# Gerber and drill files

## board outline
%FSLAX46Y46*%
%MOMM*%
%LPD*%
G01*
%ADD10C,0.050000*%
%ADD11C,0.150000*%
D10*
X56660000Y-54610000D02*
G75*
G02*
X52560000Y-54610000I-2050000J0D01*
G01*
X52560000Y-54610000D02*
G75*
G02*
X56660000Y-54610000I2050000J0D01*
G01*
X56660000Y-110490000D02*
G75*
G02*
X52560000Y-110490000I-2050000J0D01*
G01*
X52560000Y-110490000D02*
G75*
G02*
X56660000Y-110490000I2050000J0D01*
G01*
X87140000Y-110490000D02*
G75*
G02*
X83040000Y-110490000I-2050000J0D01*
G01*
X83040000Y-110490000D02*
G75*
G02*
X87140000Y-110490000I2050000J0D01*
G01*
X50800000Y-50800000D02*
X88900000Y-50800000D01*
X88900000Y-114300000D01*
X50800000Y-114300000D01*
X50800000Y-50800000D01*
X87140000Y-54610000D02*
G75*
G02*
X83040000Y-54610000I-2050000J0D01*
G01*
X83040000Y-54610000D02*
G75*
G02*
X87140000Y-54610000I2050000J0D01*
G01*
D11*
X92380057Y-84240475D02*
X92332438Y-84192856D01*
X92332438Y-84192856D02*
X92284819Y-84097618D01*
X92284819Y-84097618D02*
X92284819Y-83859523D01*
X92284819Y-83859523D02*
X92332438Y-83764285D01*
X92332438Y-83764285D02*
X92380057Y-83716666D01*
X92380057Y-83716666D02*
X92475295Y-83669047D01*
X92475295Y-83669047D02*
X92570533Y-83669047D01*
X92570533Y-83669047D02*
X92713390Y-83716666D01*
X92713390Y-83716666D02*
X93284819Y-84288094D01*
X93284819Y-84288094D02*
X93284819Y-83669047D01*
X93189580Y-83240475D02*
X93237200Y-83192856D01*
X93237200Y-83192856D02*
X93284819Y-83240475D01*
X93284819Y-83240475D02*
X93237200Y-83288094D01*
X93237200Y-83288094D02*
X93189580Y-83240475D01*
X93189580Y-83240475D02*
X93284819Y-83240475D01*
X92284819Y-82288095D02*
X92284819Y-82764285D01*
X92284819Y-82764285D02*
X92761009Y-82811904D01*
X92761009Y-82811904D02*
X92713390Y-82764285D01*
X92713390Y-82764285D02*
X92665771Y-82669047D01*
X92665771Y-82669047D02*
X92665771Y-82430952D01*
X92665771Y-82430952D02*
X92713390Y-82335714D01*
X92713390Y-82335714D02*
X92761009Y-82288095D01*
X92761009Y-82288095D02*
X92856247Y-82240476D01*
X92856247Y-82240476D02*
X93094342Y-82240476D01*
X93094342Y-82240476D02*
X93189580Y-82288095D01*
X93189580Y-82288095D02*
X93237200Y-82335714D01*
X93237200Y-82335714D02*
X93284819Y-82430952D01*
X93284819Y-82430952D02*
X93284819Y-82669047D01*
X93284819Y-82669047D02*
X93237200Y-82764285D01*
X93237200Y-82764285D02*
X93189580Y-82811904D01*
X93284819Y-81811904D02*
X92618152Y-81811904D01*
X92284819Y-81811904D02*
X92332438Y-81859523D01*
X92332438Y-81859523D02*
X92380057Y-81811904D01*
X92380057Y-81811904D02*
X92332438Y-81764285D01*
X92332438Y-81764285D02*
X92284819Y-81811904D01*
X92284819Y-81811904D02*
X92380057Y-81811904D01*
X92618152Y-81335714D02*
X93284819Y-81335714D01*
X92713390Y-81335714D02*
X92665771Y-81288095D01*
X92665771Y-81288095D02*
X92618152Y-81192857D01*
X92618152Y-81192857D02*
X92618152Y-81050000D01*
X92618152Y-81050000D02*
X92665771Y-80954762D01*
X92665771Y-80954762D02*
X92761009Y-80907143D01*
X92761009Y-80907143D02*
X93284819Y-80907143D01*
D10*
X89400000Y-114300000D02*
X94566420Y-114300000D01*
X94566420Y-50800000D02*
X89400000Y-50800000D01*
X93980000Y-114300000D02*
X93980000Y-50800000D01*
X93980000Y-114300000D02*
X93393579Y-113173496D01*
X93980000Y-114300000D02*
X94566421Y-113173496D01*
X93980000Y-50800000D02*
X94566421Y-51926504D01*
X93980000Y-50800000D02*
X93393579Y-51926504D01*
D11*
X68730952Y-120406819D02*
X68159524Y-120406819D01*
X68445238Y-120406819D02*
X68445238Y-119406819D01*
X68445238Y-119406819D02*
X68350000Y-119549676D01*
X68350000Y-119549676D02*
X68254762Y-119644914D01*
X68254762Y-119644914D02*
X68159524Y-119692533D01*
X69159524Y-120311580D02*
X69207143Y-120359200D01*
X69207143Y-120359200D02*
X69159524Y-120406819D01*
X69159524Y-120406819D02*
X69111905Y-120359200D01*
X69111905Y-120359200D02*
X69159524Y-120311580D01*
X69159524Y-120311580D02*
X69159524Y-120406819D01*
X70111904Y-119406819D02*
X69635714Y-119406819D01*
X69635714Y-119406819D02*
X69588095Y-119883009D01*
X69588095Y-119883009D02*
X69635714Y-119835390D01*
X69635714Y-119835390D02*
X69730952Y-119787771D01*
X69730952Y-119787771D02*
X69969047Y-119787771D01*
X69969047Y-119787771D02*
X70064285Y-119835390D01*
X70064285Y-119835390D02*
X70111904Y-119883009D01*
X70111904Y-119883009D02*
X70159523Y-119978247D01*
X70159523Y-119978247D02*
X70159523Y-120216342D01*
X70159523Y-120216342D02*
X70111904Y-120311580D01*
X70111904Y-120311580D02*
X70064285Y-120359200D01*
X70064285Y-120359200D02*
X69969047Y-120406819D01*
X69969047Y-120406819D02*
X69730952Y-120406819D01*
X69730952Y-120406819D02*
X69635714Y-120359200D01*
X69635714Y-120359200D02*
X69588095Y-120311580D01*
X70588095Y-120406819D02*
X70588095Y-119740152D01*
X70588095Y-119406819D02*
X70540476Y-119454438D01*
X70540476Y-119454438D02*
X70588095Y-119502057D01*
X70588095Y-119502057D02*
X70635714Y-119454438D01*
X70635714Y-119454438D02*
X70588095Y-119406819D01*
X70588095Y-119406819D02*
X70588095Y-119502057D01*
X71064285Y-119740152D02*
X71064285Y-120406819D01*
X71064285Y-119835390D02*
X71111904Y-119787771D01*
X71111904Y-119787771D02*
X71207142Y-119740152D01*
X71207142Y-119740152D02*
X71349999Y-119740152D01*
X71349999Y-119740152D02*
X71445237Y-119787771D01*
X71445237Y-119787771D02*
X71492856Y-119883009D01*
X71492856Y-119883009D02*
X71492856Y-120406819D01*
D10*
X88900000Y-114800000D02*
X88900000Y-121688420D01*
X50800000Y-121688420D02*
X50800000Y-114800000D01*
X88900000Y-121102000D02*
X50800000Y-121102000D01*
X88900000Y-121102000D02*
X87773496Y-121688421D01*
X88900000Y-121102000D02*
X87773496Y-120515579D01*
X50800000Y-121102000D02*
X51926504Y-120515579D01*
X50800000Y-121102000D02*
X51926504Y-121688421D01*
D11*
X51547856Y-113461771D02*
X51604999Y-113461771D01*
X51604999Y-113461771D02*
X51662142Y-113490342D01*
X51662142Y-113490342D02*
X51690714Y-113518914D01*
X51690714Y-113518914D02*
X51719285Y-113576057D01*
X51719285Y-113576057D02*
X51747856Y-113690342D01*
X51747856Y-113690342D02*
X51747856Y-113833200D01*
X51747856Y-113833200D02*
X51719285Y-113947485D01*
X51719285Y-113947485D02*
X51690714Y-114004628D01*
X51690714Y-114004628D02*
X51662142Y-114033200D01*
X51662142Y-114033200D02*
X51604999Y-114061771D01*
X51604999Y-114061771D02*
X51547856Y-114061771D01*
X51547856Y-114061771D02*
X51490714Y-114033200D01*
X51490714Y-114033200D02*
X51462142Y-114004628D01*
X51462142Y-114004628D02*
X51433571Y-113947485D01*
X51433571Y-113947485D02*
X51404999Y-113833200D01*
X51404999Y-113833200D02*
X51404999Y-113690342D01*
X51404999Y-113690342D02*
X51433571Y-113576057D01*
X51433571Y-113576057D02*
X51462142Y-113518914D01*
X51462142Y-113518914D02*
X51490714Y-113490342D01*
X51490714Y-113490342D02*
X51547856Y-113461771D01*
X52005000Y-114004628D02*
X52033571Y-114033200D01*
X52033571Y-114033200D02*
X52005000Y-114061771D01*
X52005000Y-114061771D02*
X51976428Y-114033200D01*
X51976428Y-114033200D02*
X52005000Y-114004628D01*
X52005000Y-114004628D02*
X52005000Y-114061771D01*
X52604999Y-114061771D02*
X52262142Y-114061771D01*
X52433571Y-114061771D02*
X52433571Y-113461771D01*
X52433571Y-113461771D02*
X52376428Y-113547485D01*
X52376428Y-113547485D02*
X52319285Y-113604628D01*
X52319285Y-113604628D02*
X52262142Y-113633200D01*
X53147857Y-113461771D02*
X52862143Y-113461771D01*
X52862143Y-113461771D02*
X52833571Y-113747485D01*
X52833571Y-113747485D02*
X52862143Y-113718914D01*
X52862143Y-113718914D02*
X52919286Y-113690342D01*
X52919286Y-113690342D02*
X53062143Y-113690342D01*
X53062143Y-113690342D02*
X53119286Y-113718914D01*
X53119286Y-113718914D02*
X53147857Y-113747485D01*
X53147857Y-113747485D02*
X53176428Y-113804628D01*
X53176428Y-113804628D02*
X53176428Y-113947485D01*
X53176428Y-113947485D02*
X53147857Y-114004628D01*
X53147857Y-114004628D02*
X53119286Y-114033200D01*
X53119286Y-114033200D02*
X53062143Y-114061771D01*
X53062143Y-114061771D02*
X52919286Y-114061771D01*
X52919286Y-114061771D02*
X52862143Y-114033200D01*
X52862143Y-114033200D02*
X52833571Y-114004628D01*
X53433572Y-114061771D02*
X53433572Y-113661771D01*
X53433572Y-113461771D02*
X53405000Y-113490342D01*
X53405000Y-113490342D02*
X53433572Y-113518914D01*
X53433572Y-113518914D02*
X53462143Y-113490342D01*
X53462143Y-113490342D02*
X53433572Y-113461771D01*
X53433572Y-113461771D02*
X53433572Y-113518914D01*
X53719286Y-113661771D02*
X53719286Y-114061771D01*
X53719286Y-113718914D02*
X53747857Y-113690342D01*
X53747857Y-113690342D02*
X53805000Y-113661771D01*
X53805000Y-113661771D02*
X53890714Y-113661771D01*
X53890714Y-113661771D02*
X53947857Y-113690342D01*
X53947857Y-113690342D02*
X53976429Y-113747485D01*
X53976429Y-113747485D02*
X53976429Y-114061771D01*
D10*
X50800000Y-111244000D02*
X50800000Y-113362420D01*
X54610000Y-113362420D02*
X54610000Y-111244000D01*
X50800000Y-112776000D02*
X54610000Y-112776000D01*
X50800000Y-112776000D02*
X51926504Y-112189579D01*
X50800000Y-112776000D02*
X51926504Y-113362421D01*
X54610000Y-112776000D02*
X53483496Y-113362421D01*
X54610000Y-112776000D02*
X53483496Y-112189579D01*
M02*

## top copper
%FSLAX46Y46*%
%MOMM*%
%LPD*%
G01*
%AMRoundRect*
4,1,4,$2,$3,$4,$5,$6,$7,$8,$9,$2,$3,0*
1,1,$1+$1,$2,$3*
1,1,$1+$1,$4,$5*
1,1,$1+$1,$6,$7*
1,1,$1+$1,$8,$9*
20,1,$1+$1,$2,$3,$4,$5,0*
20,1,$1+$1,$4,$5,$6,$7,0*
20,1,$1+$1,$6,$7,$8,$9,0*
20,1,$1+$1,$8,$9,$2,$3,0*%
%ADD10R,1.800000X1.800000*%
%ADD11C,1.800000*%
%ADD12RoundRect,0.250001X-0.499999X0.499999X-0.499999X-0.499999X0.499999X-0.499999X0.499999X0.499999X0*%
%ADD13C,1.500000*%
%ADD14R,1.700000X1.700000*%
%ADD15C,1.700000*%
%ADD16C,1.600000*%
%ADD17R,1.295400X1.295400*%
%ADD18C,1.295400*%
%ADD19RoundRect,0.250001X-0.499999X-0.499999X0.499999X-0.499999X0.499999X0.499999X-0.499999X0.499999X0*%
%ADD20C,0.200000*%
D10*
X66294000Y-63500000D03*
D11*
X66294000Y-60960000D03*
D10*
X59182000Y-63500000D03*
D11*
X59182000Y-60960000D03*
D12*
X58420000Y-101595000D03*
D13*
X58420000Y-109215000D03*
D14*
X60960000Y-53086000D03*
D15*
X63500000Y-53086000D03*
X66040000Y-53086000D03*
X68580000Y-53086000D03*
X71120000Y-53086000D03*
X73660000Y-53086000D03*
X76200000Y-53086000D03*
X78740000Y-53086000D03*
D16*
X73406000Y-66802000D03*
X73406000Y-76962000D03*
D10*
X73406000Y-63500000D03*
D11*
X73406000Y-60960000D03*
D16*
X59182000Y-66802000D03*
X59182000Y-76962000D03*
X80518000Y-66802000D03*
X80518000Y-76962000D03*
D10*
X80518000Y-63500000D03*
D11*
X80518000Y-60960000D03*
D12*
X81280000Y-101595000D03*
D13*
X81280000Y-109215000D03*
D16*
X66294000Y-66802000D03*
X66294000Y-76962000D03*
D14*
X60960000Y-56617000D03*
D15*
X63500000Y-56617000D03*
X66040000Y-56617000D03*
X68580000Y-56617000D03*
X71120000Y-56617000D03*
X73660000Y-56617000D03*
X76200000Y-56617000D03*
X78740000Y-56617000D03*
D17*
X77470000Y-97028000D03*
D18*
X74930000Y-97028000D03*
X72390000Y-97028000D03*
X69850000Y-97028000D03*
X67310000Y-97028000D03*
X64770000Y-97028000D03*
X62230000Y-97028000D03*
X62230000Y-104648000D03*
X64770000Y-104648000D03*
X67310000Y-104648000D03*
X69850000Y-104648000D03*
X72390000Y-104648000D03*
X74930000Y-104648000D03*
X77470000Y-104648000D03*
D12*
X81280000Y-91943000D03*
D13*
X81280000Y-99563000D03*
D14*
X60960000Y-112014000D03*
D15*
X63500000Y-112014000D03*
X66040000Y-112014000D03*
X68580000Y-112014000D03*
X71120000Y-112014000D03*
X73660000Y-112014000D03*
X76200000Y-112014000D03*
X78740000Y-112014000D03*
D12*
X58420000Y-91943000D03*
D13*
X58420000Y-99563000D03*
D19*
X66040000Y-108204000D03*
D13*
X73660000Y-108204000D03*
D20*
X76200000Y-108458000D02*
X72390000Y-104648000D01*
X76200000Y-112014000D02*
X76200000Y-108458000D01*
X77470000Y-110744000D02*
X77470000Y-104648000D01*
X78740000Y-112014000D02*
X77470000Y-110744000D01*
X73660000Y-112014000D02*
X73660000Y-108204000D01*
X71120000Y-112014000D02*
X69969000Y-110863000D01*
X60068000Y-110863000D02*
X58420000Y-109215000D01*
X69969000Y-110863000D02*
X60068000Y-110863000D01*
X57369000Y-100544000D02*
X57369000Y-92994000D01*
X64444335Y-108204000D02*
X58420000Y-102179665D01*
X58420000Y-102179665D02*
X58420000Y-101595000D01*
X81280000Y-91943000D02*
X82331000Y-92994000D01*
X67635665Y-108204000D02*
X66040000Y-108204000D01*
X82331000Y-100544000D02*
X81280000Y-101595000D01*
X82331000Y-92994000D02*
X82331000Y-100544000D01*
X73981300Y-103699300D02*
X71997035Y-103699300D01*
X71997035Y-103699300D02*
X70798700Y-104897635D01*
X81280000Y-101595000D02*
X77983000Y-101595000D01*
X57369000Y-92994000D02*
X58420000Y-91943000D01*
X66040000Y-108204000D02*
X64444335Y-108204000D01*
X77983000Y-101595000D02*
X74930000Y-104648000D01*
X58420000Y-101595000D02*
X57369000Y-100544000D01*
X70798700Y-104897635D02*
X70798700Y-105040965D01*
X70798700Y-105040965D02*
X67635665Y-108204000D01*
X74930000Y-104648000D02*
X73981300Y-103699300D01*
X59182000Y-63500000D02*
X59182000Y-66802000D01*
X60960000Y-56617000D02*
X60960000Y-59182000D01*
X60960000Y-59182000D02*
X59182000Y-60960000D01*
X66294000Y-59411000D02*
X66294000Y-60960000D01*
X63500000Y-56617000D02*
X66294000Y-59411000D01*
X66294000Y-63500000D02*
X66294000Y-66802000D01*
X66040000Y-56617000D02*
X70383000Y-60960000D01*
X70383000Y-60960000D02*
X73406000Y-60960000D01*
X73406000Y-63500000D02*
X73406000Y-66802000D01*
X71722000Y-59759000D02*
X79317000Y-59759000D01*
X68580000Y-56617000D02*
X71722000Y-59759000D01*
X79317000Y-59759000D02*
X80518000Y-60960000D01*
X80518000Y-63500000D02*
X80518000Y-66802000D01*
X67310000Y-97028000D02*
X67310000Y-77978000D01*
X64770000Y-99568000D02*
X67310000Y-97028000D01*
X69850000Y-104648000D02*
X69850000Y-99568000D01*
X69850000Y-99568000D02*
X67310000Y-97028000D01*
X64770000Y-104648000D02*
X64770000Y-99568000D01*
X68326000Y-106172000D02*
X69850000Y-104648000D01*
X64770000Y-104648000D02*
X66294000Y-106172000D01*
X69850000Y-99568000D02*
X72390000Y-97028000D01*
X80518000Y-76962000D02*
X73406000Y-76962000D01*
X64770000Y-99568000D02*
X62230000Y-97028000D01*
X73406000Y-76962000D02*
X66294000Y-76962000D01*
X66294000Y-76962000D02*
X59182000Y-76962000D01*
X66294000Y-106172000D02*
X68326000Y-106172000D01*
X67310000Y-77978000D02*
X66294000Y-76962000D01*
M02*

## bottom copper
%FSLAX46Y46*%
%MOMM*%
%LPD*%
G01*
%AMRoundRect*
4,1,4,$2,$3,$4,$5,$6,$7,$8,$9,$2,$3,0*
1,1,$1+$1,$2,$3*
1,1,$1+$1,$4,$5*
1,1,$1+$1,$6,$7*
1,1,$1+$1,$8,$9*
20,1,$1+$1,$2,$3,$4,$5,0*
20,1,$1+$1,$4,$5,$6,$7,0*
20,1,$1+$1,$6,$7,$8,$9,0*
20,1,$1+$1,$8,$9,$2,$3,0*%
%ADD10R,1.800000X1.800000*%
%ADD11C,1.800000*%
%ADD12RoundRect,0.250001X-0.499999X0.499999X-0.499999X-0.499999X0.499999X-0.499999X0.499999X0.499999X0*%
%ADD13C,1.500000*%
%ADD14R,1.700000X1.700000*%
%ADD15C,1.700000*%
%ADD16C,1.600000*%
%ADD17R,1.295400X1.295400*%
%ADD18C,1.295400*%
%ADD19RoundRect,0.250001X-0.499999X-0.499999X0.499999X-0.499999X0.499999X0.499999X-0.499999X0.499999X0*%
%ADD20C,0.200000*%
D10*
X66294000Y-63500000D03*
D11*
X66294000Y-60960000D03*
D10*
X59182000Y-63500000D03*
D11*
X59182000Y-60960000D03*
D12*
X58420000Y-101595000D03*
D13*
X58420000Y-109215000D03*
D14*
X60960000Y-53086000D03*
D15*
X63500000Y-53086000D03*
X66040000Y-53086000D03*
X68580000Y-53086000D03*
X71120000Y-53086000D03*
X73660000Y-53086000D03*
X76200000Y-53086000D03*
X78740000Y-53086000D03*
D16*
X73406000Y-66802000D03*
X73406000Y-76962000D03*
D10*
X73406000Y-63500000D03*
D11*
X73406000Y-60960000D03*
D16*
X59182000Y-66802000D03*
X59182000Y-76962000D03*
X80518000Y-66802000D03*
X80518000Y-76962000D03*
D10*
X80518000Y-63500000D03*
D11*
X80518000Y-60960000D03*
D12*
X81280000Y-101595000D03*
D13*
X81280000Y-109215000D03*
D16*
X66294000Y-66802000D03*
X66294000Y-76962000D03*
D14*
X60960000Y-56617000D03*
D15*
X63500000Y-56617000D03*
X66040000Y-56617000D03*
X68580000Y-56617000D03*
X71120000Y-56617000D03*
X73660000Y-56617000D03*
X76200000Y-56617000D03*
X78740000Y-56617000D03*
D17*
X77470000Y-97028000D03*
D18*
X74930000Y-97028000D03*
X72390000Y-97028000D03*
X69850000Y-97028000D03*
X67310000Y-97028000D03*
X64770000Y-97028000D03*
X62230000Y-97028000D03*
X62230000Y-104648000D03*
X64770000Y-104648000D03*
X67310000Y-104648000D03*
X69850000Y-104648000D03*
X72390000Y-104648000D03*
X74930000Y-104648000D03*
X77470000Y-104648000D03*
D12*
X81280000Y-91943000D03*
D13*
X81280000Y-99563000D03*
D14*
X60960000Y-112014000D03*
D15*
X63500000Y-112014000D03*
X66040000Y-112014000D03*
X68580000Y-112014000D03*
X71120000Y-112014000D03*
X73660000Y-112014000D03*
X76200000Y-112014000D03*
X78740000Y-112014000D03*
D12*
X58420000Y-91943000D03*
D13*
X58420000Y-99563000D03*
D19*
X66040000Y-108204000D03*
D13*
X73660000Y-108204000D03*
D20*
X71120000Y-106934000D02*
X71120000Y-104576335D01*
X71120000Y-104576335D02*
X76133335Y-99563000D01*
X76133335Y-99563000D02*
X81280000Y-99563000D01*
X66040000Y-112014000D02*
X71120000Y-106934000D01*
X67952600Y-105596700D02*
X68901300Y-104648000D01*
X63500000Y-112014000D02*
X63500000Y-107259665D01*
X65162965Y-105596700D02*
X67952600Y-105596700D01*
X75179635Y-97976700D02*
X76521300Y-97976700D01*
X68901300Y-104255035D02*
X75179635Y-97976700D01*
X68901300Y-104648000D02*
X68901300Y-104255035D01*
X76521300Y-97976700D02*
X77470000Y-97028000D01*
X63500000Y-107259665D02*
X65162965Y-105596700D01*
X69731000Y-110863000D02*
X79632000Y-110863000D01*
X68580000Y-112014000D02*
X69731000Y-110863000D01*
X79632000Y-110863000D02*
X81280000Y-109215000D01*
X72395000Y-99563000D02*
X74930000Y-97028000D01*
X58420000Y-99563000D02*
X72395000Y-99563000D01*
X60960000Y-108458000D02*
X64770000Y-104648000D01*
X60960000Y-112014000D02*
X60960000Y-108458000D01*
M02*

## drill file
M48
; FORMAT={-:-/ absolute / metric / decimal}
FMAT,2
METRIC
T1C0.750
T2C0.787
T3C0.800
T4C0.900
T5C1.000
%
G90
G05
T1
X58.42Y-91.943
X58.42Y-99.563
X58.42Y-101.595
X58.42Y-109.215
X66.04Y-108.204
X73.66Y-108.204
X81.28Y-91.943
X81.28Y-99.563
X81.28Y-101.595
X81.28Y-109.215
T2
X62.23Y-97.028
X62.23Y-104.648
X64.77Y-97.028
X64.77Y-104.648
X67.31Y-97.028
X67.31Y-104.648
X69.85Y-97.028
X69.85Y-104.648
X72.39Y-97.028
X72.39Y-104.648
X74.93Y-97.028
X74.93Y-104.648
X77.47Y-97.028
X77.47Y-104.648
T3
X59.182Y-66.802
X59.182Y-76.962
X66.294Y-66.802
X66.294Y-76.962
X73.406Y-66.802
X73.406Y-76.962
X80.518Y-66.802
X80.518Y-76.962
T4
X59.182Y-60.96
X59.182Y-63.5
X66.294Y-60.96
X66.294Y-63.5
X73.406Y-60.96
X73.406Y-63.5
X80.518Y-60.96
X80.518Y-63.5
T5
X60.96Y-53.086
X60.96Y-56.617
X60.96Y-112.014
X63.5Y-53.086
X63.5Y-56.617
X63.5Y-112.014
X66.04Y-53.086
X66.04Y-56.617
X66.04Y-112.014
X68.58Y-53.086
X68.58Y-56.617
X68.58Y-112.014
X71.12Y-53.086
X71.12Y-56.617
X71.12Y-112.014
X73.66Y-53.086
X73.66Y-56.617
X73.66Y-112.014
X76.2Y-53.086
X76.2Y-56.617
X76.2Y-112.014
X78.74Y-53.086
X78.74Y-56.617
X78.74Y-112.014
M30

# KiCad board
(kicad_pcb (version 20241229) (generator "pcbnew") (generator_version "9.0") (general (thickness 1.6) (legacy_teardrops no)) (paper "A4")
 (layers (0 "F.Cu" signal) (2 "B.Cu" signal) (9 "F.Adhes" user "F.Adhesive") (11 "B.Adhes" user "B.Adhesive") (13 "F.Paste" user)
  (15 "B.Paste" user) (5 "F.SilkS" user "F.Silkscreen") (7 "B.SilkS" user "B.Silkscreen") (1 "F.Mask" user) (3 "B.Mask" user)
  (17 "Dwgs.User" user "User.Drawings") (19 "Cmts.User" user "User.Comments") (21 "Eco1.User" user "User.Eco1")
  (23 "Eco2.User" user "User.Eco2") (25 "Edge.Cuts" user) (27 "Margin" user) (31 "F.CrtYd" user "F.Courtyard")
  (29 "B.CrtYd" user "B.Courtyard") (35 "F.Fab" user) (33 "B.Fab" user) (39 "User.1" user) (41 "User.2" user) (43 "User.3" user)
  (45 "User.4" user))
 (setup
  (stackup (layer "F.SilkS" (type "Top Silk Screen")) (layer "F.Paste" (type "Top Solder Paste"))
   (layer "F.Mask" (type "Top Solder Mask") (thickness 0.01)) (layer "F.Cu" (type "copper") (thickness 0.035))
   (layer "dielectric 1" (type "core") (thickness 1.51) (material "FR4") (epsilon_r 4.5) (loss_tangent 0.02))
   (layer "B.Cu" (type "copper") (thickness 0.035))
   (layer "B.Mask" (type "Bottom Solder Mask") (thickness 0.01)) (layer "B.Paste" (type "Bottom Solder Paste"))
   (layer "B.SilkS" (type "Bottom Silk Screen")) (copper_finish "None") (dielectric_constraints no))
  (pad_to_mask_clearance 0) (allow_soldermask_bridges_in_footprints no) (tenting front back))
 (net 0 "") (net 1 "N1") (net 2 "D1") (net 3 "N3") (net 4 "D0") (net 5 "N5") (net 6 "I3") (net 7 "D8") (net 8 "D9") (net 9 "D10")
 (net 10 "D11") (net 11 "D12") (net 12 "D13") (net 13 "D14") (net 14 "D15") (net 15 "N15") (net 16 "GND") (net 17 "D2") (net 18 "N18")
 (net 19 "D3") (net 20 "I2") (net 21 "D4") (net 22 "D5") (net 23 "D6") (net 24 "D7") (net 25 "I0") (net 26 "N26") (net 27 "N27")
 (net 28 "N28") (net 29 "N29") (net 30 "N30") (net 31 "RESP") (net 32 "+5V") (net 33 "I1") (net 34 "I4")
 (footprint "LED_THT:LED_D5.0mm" (layer "F.Cu") (at 66.294 63.5 90)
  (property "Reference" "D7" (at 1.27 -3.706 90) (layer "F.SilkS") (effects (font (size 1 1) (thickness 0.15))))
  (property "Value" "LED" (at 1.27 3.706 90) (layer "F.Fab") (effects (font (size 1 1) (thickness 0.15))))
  (pad "1" thru_hole rect (at 0 0 90) (size 1.8 1.8) (drill 0.9) (layers "*.Cu" "*.Mask") (remove_unused_layers no) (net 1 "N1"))
  (pad "2" thru_hole circle (at 2.54 0 90) (size 1.8 1.8) (drill 0.9) (layers "*.Cu" "*.Mask") (remove_unused_layers no) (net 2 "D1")))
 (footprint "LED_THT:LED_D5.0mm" (layer "F.Cu") (at 59.182 63.5 90)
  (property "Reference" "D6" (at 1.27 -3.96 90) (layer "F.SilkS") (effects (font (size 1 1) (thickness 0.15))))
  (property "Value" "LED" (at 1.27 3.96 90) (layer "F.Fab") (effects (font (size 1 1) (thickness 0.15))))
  (pad "1" thru_hole rect (at 0 0 90) (size 1.8 1.8) (drill 0.9) (layers "*.Cu" "*.Mask") (remove_unused_layers no) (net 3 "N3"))
  (pad "2" thru_hole circle (at 2.54 0 90) (size 1.8 1.8) (drill 0.9) (layers "*.Cu" "*.Mask") (remove_unused_layers no) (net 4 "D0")))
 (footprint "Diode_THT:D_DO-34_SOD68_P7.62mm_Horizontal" (layer "F.Cu") (at 58.42 101.595 -90)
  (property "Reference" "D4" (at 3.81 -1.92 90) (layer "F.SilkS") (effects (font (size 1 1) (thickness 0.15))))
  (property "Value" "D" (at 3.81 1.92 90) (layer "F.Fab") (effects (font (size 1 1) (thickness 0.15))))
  (pad "1" thru_hole roundrect (at 0 0 270) (size 1.5 1.5) (drill 0.75) (layers "*.Cu" "*.Mask") (remove_unused_layers no)
   (roundrect_rratio 0.166667) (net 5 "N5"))
  (pad "2" thru_hole circle (at 7.62 0 270) (size 1.5 1.5) (drill 0.75) (layers "*.Cu" "*.Mask") (remove_unused_layers no) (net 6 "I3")))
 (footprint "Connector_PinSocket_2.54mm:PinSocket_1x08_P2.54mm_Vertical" (layer "F.Cu") (at 60.96 53.086 90)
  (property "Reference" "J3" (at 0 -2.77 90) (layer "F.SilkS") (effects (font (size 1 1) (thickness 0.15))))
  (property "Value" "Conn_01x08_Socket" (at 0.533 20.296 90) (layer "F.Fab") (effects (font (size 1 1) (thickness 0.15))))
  (pad "1" thru_hole rect (at 0 0 90) (size 1.7 1.7) (drill 1) (layers "*.Cu" "*.Mask") (remove_unused_layers no) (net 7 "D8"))
  (pad "2" thru_hole circle (at 0 2.54 90) (size 1.7 1.7) (drill 1) (layers "*.Cu" "*.Mask") (remove_unused_layers no) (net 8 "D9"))
  (pad "3" thru_hole circle (at 0 5.08 90) (size 1.7 1.7) (drill 1) (layers "*.Cu" "*.Mask") (remove_unused_layers no) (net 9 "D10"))
  (pad "4" thru_hole circle (at 0 7.62 90) (size 1.7 1.7) (drill 1) (layers "*.Cu" "*.Mask") (remove_unused_layers no) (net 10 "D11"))
  (pad "5" thru_hole circle (at 0 10.16 90) (size 1.7 1.7) (drill 1) (layers "*.Cu" "*.Mask") (remove_unused_layers no) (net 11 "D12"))
  (pad "6" thru_hole circle (at 0 12.7 90) (size 1.7 1.7) (drill 1) (layers "*.Cu" "*.Mask") (remove_unused_layers no) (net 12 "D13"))
  (pad "7" thru_hole circle (at 0 15.24 90) (size 1.7 1.7) (drill 1) (layers "*.Cu" "*.Mask") (remove_unused_layers no) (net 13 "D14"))
  (pad "8" thru_hole circle (at 0 17.78 90) (size 1.7 1.7) (drill 1) (layers "*.Cu" "*.Mask") (remove_unused_layers no) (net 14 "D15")))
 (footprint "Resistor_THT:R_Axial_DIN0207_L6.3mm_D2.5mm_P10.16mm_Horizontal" (layer "F.Cu") (at 73.406 66.802 -90)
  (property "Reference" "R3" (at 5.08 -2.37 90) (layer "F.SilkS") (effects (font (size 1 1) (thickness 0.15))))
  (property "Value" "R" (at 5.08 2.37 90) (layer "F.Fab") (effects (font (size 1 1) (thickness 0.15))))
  (pad "1" thru_hole circle (at 0 0 270) (size 1.6 1.6) (drill 0.8) (layers "*.Cu" "*.Mask") (remove_unused_layers no) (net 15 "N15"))
  (pad "2" thru_hole circle (at 10.16 0 270) (size 1.6 1.6) (drill 0.8) (layers "*.Cu" "*.Mask") (remove_unused_layers no) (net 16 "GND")))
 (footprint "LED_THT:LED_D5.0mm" (layer "F.Cu") (at 73.406 63.5 90)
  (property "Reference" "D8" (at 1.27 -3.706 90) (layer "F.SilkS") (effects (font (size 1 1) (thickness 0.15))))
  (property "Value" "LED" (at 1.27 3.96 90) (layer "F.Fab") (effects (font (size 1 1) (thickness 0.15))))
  (pad "1" thru_hole rect (at 0 0 90) (size 1.8 1.8) (drill 0.9) (layers "*.Cu" "*.Mask") (remove_unused_layers no) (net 15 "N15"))
  (pad "2" thru_hole circle (at 2.54 0 90) (size 1.8 1.8) (drill 0.9) (layers "*.Cu" "*.Mask") (remove_unused_layers no) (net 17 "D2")))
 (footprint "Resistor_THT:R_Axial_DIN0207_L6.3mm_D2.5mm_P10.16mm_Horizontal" (layer "F.Cu") (at 59.182 66.802 -90)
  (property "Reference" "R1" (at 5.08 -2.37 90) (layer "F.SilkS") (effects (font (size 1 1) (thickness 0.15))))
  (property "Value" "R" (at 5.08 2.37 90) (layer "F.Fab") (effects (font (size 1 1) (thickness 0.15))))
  (pad "1" thru_hole circle (at 0 0 270) (size 1.6 1.6) (drill 0.8) (layers "*.Cu" "*.Mask") (remove_unused_layers no) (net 3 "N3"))
  (pad "2" thru_hole circle (at 10.16 0 270) (size 1.6 1.6) (drill 0.8) (layers "*.Cu" "*.Mask") (remove_unused_layers no) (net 16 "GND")))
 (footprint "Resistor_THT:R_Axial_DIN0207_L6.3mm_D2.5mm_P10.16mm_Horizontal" (layer "F.Cu") (at 80.518 66.802 -90)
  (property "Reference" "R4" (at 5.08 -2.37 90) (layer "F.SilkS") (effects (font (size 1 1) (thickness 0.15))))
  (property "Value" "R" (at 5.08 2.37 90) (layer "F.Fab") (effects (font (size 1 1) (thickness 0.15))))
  (pad "1" thru_hole circle (at 0 0 270) (size 1.6 1.6) (drill 0.8) (layers "*.Cu" "*.Mask") (remove_unused_layers no) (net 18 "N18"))
  (pad "2" thru_hole circle (at 10.16 0 270) (size 1.6 1.6) (drill 0.8) (layers "*.Cu" "*.Mask") (remove_unused_layers no) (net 16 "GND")))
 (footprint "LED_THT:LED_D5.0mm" (layer "F.Cu") (at 80.518 63.5 90)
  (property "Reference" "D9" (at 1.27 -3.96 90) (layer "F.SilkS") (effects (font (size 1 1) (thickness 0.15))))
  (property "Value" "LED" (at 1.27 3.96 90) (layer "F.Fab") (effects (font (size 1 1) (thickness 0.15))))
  (pad "1" thru_hole rect (at 0 0 90) (size 1.8 1.8) (drill 0.9) (layers "*.Cu" "*.Mask") (remove_unused_layers no) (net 18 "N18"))
  (pad "2" thru_hole circle (at 2.54 0 90) (size 1.8 1.8) (drill 0.9) (layers "*.Cu" "*.Mask") (remove_unused_layers no) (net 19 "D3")))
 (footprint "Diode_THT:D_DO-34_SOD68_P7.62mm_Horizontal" (layer "F.Cu") (at 81.28 101.595 -90)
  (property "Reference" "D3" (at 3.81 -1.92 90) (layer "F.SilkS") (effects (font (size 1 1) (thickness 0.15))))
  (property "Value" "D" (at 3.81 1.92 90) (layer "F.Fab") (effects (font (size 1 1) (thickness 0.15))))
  (pad "1" thru_hole roundrect (at 0 0 270) (size 1.5 1.5) (drill 0.75) (layers "*.Cu" "*.Mask") (remove_unused_layers no)
   (roundrect_rratio 0.166667) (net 5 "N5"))
  (pad "2" thru_hole circle (at 7.62 0 270) (size 1.5 1.5) (drill 0.75) (layers "*.Cu" "*.Mask") (remove_unused_layers no) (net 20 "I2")))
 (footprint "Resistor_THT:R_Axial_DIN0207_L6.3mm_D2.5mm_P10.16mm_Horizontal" (layer "F.Cu") (at 66.294 66.802 -90)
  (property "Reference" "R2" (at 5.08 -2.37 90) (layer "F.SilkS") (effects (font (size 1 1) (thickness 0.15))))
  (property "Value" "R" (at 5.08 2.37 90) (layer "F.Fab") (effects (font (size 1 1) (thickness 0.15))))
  (pad "1" thru_hole circle (at 0 0 270) (size 1.6 1.6) (drill 0.8) (layers "*.Cu" "*.Mask") (remove_unused_layers no) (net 1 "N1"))
  (pad "2" thru_hole circle (at 10.16 0 270) (size 1.6 1.6) (drill 0.8) (layers "*.Cu" "*.Mask") (remove_unused_layers no) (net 16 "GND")))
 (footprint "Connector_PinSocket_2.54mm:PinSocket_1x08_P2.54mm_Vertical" (layer "F.Cu") (at 60.96 56.617 90)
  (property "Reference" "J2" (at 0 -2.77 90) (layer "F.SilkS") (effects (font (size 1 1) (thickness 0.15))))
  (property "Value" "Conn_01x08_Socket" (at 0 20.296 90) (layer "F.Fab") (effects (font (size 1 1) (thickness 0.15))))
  (pad "1" thru_hole rect (at 0 0 90) (size 1.7 1.7) (drill 1) (layers "*.Cu" "*.Mask") (remove_unused_layers no) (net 4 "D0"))
  (pad "2" thru_hole circle (at 0 2.54 90) (size 1.7 1.7) (drill 1) (layers "*.Cu" "*.Mask") (remove_unused_layers no) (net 2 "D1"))
  (pad "3" thru_hole circle (at 0 5.08 90) (size 1.7 1.7) (drill 1) (layers "*.Cu" "*.Mask") (remove_unused_layers no) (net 17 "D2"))
  (pad "4" thru_hole circle (at 0 7.62 90) (size 1.7 1.7) (drill 1) (layers "*.Cu" "*.Mask") (remove_unused_layers no) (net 19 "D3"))
  (pad "5" thru_hole circle (at 0 10.16 90) (size 1.7 1.7) (drill 1) (layers "*.Cu" "*.Mask") (remove_unused_layers no) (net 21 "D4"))
  (pad "6" thru_hole circle (at 0 12.7 90) (size 1.7 1.7) (drill 1) (layers "*.Cu" "*.Mask") (remove_unused_layers no) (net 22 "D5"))
  (pad "7" thru_hole circle (at 0 15.24 90) (size 1.7 1.7) (drill 1) (layers "*.Cu" "*.Mask") (remove_unused_layers no) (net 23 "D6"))
  (pad "8" thru_hole circle (at 0 17.78 90) (size 1.7 1.7) (drill 1) (layers "*.Cu" "*.Mask") (remove_unused_layers no) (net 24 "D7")))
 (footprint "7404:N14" (layer "F.Cu") (at 62.23 104.648 -90)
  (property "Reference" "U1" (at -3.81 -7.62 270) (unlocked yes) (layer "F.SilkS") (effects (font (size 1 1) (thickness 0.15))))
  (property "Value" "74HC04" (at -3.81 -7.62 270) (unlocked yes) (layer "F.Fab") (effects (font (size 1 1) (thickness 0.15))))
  (pad "1" thru_hole rect (at -7.62 -15.24 270) (size 1.2954 1.2954) (drill 0.7874) (layers "*.Cu" "*.Mask") (remove_unused_layers no)
   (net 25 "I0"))
  (pad "2" thru_hole circle (at -7.62 -12.7 270) (size 1.2954 1.2954) (drill 0.7874) (layers "*.Cu" "*.Mask") (remove_unused_layers no)
   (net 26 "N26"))
  (pad "3" thru_hole circle (at -7.62 -10.16 270) (size 1.2954 1.2954) (drill 0.7874) (layers "*.Cu" "*.Mask") (remove_unused_layers no)
   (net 16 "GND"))
  (pad "4" thru_hole circle (at -7.62 -7.62 270) (size 1.2954 1.2954) (drill 0.7874) (layers "*.Cu" "*.Mask") (remove_unused_layers no)
   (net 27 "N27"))
  (pad "5" thru_hole circle (at -7.62 -5.08 270) (size 1.2954 1.2954) (drill 0.7874) (layers "*.Cu" "*.Mask") (remove_unused_layers no)
   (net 16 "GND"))
  (pad "6" thru_hole circle (at -7.62 -2.54 270) (size 1.2954 1.2954) (drill 0.7874) (layers "*.Cu" "*.Mask") (remove_unused_layers no)
   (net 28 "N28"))
  (pad "7" thru_hole circle (at -7.62 0 270) (size 1.2954 1.2954) (drill 0.7874) (layers "*.Cu" "*.Mask") (remove_unused_layers no)
   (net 16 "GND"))
  (pad "8" thru_hole circle (at 0 0 270) (size 1.2954 1.2954) (drill 0.7874) (layers "*.Cu" "*.Mask") (remove_unused_layers no)
   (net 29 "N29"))
  (pad "9" thru_hole circle (at 0 -2.54 270) (size 1.2954 1.2954) (drill 0.7874) (layers "*.Cu" "*.Mask") (remove_unused_layers no)
   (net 16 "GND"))
  (pad "10" thru_hole circle (at 0 -5.08 270) (size 1.2954 1.2954) (drill 0.7874) (layers "*.Cu" "*.Mask") (remove_unused_layers no)
   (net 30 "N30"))
  (pad "11" thru_hole circle (at 0 -7.62 270) (size 1.2954 1.2954) (drill 0.7874) (layers "*.Cu" "*.Mask") (remove_unused_layers no)
   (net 16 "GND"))
  (pad "12" thru_hole circle (at 0 -10.16 270) (size 1.2954 1.2954) (drill 0.7874) (layers "*.Cu" "*.Mask") (remove_unused_layers no)
   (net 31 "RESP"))
  (pad "13" thru_hole circle (at 0 -12.7 270) (size 1.2954 1.2954) (drill 0.7874) (layers "*.Cu" "*.Mask") (remove_unused_layers no)
   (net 5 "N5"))
  (pad "14" thru_hole circle (at 0 -15.24 270) (size 1.2954 1.2954) (drill 0.7874) (layers "*.Cu" "*.Mask") (remove_unused_layers no)
   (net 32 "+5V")))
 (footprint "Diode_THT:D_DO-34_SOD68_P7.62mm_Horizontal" (layer "F.Cu") (at 81.28 91.943 -90)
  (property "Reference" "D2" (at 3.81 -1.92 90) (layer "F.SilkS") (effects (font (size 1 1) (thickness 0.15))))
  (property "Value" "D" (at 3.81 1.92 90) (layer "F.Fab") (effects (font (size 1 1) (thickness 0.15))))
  (pad "1" thru_hole roundrect (at 0 0 270) (size 1.5 1.5) (drill 0.75) (layers "*.Cu" "*.Mask") (remove_unused_layers no)
   (roundrect_rratio 0.166667) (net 5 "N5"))
  (pad "2" thru_hole circle (at 7.62 0 270) (size 1.5 1.5) (drill 0.75) (layers "*.Cu" "*.Mask") (remove_unused_layers no) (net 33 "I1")))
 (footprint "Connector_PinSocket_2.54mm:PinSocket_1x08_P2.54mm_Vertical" (layer "F.Cu") (at 60.96 112.014 90)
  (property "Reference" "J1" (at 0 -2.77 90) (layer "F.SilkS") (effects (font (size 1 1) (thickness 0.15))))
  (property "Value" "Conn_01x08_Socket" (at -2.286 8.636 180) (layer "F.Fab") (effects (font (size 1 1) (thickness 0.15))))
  (pad "1" thru_hole rect (at 0 0 90) (size 1.7 1.7) (drill 1) (layers "*.Cu" "*.Mask") (remove_unused_layers no) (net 16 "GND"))
  (pad "2" thru_hole circle (at 0 2.54 90) (size 1.7 1.7) (drill 1) (layers "*.Cu" "*.Mask") (remove_unused_layers no) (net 25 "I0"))
  (pad "3" thru_hole circle (at 0 5.08 90) (size 1.7 1.7) (drill 1) (layers "*.Cu" "*.Mask") (remove_unused_layers no) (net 33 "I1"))
  (pad "4" thru_hole circle (at 0 7.62 90) (size 1.7 1.7) (drill 1) (layers "*.Cu" "*.Mask") (remove_unused_layers no) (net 20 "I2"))
  (pad "5" thru_hole circle (at 0 10.16 90) (size 1.7 1.7) (drill 1) (layers "*.Cu" "*.Mask") (remove_unused_layers no) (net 6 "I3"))
  (pad "6" thru_hole circle (at 0 12.7 90) (size 1.7 1.7) (drill 1) (layers "*.Cu" "*.Mask") (remove_unused_layers no) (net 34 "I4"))
  (pad "7" thru_hole circle (at 0 15.24 90) (size 1.7 1.7) (drill 1) (layers "*.Cu" "*.Mask") (remove_unused_layers no) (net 31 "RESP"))
  (pad "8" thru_hole circle (at 0 17.78 90) (size 1.7 1.7) (drill 1) (layers "*.Cu" "*.Mask") (remove_unused_layers no) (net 32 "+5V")))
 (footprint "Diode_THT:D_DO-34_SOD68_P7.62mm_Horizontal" (layer "F.Cu") (at 58.42 91.943 -90)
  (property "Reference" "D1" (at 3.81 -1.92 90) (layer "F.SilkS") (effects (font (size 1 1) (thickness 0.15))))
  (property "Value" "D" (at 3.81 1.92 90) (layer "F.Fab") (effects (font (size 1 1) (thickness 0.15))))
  (pad "1" thru_hole roundrect (at 0 0 270) (size 1.5 1.5) (drill 0.75) (layers "*.Cu" "*.Mask") (remove_unused_layers no)
   (roundrect_rratio 0.166667) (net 5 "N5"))
  (pad "2" thru_hole circle (at 7.62 0 270) (size 1.5 1.5) (drill 0.75) (layers "*.Cu" "*.Mask") (remove_unused_layers no) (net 26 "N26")))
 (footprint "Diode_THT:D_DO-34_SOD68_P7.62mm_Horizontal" (layer "F.Cu") (at 66.04 108.204)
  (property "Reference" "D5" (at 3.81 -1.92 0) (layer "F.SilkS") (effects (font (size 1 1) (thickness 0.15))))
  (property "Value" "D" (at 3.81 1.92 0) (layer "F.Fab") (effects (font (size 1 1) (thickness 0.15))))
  (pad "1" thru_hole roundrect (at 0 0) (size 1.5 1.5) (drill 0.75) (layers "*.Cu" "*.Mask") (remove_unused_layers no)
   (roundrect_rratio 0.166667) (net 5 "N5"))
  (pad "2" thru_hole circle (at 7.62 0) (size 1.5 1.5) (drill 0.75) (layers "*.Cu" "*.Mask") (remove_unused_layers no) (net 34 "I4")))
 (gr_circle (center 54.61 54.61) (end 56.66 54.61) (stroke (width 0.05) (type solid)) (fill no) (layer "Edge.Cuts"))
 (gr_circle (center 54.61 110.49) (end 56.66 110.49) (stroke (width 0.05) (type solid)) (fill no) (layer "Edge.Cuts"))
 (gr_circle (center 85.09 110.49) (end 87.14 110.49) (stroke (width 0.05) (type solid)) (fill no) (layer "Edge.Cuts"))
 (gr_rect (start 50.8 50.8) (end 88.9 114.3) (stroke (width 0.05) (type solid)) (fill no) (layer "Edge.Cuts"))
 (gr_circle (center 85.09 54.61) (end 87.14 54.61) (stroke (width 0.05) (type solid)) (fill no) (layer "Edge.Cuts"))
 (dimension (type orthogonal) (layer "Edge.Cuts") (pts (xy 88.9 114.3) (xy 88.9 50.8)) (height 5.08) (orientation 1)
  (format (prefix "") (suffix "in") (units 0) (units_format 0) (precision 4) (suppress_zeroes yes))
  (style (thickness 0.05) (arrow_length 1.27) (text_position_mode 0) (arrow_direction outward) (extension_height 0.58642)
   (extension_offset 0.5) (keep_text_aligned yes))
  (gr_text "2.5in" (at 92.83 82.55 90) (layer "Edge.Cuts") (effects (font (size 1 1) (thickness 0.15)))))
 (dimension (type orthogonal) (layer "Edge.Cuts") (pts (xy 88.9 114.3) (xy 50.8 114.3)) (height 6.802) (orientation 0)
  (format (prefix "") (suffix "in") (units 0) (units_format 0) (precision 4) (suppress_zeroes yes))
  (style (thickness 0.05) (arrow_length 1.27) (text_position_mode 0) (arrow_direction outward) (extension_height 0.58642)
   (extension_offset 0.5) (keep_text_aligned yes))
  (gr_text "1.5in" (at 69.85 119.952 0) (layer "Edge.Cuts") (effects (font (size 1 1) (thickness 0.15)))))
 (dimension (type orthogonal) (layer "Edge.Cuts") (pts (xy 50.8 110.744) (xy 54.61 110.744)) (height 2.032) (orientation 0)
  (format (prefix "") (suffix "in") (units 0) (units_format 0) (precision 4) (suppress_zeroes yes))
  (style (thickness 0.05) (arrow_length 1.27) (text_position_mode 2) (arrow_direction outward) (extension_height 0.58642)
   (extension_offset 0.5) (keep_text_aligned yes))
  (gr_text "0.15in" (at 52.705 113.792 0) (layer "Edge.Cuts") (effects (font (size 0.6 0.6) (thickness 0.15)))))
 (segment (start 71.12 106.934) (end 71.12 104.576335) (width 0.2) (layer "B.Cu") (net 33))
 (segment (start 71.12 104.576335) (end 76.133335 99.563) (width 0.2) (layer "B.Cu") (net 33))
 (segment (start 76.133335 99.563) (end 81.28 99.563) (width 0.2) (layer "B.Cu") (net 33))
 (segment (start 66.04 112.014) (end 71.12 106.934) (width 0.2) (layer "B.Cu") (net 33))
 (segment (start 76.2 108.458) (end 72.39 104.648) (width 0.2) (layer "F.Cu") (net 31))
 (segment (start 76.2 112.014) (end 76.2 108.458) (width 0.2) (layer "F.Cu") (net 31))
 (segment (start 67.9526 105.5967) (end 68.9013 104.648) (width 0.2) (layer "B.Cu") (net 25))
 (segment (start 63.5 112.014) (end 63.5 107.259665) (width 0.2) (layer "B.Cu") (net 25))
 (segment (start 65.162965 105.5967) (end 67.9526 105.5967) (width 0.2) (layer "B.Cu") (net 25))
 (segment (start 75.179635 97.9767) (end 76.5213 97.9767) (width 0.2) (layer "B.Cu") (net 25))
 (segment (start 68.9013 104.255035) (end 75.179635 97.9767) (width 0.2) (layer "B.Cu") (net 25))
 (segment (start 68.9013 104.648) (end 68.9013 104.255035) (width 0.2) (layer "B.Cu") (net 25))
 (segment (start 76.5213 97.9767) (end 77.47 97.028) (width 0.2) (layer "B.Cu") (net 25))
 (segment (start 63.5 107.259665) (end 65.162965 105.5967) (width 0.2) (layer "B.Cu") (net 25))
 (segment (start 77.47 110.744) (end 77.47 104.648) (width 0.2) (layer "F.Cu") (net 32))
 (segment (start 78.74 112.014) (end 77.47 110.744) (width 0.2) (layer "F.Cu") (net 32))
 (segment (start 73.66 112.014) (end 73.66 108.204) (width 0.2) (layer "F.Cu") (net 34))
 (segment (start 71.12 112.014) (end 69.969 110.863) (width 0.2) (layer "F.Cu") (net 6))
 (segment (start 60.068 110.863) (end 58.42 109.215) (width 0.2) (layer "F.Cu") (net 6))
 (segment (start 69.969 110.863) (end 60.068 110.863) (width 0.2) (layer "F.Cu") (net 6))
 (segment (start 69.731 110.863) (end 79.632 110.863) (width 0.2) (layer "B.Cu") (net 20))
 (segment (start 68.58 112.014) (end 69.731 110.863) (width 0.2) (layer "B.Cu") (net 20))
 (segment (start 79.632 110.863) (end 81.28 109.215) (width 0.2) (layer "B.Cu") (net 20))
 (segment (start 72.395 99.563) (end 74.93 97.028) (width 0.2) (layer "B.Cu") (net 26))
 (segment (start 58.42 99.563) (end 72.395 99.563) (width 0.2) (layer "B.Cu") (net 26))
 (segment (start 57.369 100.544) (end 57.369 92.994) (width 0.2) (layer "F.Cu") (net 5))
 (segment (start 64.444335 108.204) (end 58.42 102.179665) (width 0.2) (layer "F.Cu") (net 5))
 (segment (start 58.42 102.179665) (end 58.42 101.595) (width 0.2) (layer "F.Cu") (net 5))
 (segment (start 81.28 91.943) (end 82.331 92.994) (width 0.2) (layer "F.Cu") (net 5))
 (segment (start 67.635665 108.204) (end 66.04 108.204) (width 0.2) (layer "F.Cu") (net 5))
 (segment (start 82.331 100.544) (end 81.28 101.595) (width 0.2) (layer "F.Cu") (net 5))
 (segment (start 82.331 92.994) (end 82.331 100.544) (width 0.2) (layer "F.Cu") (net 5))
 (segment (start 73.9813 103.6993) (end 71.997035 103.6993) (width 0.2) (layer "F.Cu") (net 5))
 (segment (start 71.997035 103.6993) (end 70.7987 104.897635) (width 0.2) (layer "F.Cu") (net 5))
 (segment (start 81.28 101.595) (end 77.983 101.595) (width 0.2) (layer "F.Cu") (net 5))
 (segment (start 57.369 92.994) (end 58.42 91.943) (width 0.2) (layer "F.Cu") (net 5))
 (segment (start 66.04 108.204) (end 64.444335 108.204) (width 0.2) (layer "F.Cu") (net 5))
 (segment (start 77.983 101.595) (end 74.93 104.648) (width 0.2) (layer "F.Cu") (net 5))
 (segment (start 58.42 101.595) (end 57.369 100.544) (width 0.2) (layer "F.Cu") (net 5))
 (segment (start 70.7987 104.897635) (end 70.7987 105.040965) (width 0.2) (layer "F.Cu") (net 5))
 (segment (start 70.7987 105.040965) (end 67.635665 108.204) (width 0.2) (layer "F.Cu") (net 5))
 (segment (start 74.93 104.648) (end 73.9813 103.6993) (width 0.2) (layer "F.Cu") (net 5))
 (segment (start 59.182 63.5) (end 59.182 66.802) (width 0.2) (layer "F.Cu") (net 3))
 (segment (start 60.96 56.617) (end 60.96 59.182) (width 0.2) (layer "F.Cu") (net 4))
 (segment (start 60.96 59.182) (end 59.182 60.96) (width 0.2) (layer "F.Cu") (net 4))
 (segment (start 66.294 59.411) (end 66.294 60.96) (width 0.2) (layer "F.Cu") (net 2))
 (segment (start 63.5 56.617) (end 66.294 59.411) (width 0.2) (layer "F.Cu") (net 2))
 (segment (start 66.294 63.5) (end 66.294 66.802) (width 0.2) (layer "F.Cu") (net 1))
 (segment (start 66.04 56.617) (end 70.383 60.96) (width 0.2) (layer "F.Cu") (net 17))
 (segment (start 70.383 60.96) (end 73.406 60.96) (width 0.2) (layer "F.Cu") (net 17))
 (segment (start 73.406 63.5) (end 73.406 66.802) (width 0.2) (layer "F.Cu") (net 15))
 (segment (start 71.722 59.759) (end 79.317 59.759) (width 0.2) (layer "F.Cu") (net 19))
 (segment (start 68.58 56.617) (end 71.722 59.759) (width 0.2) (layer "F.Cu") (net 19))
 (segment (start 79.317 59.759) (end 80.518 60.96) (width 0.2) (layer "F.Cu") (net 19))
 (segment (start 80.518 63.5) (end 80.518 66.802) (width 0.2) (layer "F.Cu") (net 18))
 (segment (start 67.31 97.028) (end 67.31 77.978) (width 0.2) (layer "F.Cu") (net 16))
 (segment (start 64.77 99.568) (end 67.31 97.028) (width 0.2) (layer "F.Cu") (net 16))
 (segment (start 69.85 104.648) (end 69.85 99.568) (width 0.2) (layer "F.Cu") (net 16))
 (segment (start 69.85 99.568) (end 67.31 97.028) (width 0.2) (layer "F.Cu") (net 16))
 (segment (start 64.77 104.648) (end 64.77 99.568) (width 0.2) (layer "F.Cu") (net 16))
 (segment (start 68.326 106.172) (end 69.85 104.648) (width 0.2) (layer "F.Cu") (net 16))
 (segment (start 64.77 104.648) (end 66.294 106.172) (width 0.2) (layer "F.Cu") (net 16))
 (segment (start 69.85 99.568) (end 72.39 97.028) (width 0.2) (layer "F.Cu") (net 16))
 (segment (start 80.518 76.962) (end 73.406 76.962) (width 0.2) (layer "F.Cu") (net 16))
 (segment (start 64.77 99.568) (end 62.23 97.028) (width 0.2) (layer "F.Cu") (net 16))
 (segment (start 73.406 76.962) (end 66.294 76.962) (width 0.2) (layer "F.Cu") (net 16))
 (segment (start 66.294 76.962) (end 59.182 76.962) (width 0.2) (layer "F.Cu") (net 16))
 (segment (start 66.294 106.172) (end 68.326 106.172) (width 0.2) (layer "F.Cu") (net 16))
 (segment (start 67.31 77.978) (end 66.294 76.962) (width 0.2) (layer "F.Cu") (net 16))
 (segment (start 60.96 108.458) (end 64.77 104.648) (width 0.2) (layer "B.Cu") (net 16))
 (segment (start 60.96 112.014) (end 60.96 108.458) (width 0.2) (layer "B.Cu") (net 16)))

